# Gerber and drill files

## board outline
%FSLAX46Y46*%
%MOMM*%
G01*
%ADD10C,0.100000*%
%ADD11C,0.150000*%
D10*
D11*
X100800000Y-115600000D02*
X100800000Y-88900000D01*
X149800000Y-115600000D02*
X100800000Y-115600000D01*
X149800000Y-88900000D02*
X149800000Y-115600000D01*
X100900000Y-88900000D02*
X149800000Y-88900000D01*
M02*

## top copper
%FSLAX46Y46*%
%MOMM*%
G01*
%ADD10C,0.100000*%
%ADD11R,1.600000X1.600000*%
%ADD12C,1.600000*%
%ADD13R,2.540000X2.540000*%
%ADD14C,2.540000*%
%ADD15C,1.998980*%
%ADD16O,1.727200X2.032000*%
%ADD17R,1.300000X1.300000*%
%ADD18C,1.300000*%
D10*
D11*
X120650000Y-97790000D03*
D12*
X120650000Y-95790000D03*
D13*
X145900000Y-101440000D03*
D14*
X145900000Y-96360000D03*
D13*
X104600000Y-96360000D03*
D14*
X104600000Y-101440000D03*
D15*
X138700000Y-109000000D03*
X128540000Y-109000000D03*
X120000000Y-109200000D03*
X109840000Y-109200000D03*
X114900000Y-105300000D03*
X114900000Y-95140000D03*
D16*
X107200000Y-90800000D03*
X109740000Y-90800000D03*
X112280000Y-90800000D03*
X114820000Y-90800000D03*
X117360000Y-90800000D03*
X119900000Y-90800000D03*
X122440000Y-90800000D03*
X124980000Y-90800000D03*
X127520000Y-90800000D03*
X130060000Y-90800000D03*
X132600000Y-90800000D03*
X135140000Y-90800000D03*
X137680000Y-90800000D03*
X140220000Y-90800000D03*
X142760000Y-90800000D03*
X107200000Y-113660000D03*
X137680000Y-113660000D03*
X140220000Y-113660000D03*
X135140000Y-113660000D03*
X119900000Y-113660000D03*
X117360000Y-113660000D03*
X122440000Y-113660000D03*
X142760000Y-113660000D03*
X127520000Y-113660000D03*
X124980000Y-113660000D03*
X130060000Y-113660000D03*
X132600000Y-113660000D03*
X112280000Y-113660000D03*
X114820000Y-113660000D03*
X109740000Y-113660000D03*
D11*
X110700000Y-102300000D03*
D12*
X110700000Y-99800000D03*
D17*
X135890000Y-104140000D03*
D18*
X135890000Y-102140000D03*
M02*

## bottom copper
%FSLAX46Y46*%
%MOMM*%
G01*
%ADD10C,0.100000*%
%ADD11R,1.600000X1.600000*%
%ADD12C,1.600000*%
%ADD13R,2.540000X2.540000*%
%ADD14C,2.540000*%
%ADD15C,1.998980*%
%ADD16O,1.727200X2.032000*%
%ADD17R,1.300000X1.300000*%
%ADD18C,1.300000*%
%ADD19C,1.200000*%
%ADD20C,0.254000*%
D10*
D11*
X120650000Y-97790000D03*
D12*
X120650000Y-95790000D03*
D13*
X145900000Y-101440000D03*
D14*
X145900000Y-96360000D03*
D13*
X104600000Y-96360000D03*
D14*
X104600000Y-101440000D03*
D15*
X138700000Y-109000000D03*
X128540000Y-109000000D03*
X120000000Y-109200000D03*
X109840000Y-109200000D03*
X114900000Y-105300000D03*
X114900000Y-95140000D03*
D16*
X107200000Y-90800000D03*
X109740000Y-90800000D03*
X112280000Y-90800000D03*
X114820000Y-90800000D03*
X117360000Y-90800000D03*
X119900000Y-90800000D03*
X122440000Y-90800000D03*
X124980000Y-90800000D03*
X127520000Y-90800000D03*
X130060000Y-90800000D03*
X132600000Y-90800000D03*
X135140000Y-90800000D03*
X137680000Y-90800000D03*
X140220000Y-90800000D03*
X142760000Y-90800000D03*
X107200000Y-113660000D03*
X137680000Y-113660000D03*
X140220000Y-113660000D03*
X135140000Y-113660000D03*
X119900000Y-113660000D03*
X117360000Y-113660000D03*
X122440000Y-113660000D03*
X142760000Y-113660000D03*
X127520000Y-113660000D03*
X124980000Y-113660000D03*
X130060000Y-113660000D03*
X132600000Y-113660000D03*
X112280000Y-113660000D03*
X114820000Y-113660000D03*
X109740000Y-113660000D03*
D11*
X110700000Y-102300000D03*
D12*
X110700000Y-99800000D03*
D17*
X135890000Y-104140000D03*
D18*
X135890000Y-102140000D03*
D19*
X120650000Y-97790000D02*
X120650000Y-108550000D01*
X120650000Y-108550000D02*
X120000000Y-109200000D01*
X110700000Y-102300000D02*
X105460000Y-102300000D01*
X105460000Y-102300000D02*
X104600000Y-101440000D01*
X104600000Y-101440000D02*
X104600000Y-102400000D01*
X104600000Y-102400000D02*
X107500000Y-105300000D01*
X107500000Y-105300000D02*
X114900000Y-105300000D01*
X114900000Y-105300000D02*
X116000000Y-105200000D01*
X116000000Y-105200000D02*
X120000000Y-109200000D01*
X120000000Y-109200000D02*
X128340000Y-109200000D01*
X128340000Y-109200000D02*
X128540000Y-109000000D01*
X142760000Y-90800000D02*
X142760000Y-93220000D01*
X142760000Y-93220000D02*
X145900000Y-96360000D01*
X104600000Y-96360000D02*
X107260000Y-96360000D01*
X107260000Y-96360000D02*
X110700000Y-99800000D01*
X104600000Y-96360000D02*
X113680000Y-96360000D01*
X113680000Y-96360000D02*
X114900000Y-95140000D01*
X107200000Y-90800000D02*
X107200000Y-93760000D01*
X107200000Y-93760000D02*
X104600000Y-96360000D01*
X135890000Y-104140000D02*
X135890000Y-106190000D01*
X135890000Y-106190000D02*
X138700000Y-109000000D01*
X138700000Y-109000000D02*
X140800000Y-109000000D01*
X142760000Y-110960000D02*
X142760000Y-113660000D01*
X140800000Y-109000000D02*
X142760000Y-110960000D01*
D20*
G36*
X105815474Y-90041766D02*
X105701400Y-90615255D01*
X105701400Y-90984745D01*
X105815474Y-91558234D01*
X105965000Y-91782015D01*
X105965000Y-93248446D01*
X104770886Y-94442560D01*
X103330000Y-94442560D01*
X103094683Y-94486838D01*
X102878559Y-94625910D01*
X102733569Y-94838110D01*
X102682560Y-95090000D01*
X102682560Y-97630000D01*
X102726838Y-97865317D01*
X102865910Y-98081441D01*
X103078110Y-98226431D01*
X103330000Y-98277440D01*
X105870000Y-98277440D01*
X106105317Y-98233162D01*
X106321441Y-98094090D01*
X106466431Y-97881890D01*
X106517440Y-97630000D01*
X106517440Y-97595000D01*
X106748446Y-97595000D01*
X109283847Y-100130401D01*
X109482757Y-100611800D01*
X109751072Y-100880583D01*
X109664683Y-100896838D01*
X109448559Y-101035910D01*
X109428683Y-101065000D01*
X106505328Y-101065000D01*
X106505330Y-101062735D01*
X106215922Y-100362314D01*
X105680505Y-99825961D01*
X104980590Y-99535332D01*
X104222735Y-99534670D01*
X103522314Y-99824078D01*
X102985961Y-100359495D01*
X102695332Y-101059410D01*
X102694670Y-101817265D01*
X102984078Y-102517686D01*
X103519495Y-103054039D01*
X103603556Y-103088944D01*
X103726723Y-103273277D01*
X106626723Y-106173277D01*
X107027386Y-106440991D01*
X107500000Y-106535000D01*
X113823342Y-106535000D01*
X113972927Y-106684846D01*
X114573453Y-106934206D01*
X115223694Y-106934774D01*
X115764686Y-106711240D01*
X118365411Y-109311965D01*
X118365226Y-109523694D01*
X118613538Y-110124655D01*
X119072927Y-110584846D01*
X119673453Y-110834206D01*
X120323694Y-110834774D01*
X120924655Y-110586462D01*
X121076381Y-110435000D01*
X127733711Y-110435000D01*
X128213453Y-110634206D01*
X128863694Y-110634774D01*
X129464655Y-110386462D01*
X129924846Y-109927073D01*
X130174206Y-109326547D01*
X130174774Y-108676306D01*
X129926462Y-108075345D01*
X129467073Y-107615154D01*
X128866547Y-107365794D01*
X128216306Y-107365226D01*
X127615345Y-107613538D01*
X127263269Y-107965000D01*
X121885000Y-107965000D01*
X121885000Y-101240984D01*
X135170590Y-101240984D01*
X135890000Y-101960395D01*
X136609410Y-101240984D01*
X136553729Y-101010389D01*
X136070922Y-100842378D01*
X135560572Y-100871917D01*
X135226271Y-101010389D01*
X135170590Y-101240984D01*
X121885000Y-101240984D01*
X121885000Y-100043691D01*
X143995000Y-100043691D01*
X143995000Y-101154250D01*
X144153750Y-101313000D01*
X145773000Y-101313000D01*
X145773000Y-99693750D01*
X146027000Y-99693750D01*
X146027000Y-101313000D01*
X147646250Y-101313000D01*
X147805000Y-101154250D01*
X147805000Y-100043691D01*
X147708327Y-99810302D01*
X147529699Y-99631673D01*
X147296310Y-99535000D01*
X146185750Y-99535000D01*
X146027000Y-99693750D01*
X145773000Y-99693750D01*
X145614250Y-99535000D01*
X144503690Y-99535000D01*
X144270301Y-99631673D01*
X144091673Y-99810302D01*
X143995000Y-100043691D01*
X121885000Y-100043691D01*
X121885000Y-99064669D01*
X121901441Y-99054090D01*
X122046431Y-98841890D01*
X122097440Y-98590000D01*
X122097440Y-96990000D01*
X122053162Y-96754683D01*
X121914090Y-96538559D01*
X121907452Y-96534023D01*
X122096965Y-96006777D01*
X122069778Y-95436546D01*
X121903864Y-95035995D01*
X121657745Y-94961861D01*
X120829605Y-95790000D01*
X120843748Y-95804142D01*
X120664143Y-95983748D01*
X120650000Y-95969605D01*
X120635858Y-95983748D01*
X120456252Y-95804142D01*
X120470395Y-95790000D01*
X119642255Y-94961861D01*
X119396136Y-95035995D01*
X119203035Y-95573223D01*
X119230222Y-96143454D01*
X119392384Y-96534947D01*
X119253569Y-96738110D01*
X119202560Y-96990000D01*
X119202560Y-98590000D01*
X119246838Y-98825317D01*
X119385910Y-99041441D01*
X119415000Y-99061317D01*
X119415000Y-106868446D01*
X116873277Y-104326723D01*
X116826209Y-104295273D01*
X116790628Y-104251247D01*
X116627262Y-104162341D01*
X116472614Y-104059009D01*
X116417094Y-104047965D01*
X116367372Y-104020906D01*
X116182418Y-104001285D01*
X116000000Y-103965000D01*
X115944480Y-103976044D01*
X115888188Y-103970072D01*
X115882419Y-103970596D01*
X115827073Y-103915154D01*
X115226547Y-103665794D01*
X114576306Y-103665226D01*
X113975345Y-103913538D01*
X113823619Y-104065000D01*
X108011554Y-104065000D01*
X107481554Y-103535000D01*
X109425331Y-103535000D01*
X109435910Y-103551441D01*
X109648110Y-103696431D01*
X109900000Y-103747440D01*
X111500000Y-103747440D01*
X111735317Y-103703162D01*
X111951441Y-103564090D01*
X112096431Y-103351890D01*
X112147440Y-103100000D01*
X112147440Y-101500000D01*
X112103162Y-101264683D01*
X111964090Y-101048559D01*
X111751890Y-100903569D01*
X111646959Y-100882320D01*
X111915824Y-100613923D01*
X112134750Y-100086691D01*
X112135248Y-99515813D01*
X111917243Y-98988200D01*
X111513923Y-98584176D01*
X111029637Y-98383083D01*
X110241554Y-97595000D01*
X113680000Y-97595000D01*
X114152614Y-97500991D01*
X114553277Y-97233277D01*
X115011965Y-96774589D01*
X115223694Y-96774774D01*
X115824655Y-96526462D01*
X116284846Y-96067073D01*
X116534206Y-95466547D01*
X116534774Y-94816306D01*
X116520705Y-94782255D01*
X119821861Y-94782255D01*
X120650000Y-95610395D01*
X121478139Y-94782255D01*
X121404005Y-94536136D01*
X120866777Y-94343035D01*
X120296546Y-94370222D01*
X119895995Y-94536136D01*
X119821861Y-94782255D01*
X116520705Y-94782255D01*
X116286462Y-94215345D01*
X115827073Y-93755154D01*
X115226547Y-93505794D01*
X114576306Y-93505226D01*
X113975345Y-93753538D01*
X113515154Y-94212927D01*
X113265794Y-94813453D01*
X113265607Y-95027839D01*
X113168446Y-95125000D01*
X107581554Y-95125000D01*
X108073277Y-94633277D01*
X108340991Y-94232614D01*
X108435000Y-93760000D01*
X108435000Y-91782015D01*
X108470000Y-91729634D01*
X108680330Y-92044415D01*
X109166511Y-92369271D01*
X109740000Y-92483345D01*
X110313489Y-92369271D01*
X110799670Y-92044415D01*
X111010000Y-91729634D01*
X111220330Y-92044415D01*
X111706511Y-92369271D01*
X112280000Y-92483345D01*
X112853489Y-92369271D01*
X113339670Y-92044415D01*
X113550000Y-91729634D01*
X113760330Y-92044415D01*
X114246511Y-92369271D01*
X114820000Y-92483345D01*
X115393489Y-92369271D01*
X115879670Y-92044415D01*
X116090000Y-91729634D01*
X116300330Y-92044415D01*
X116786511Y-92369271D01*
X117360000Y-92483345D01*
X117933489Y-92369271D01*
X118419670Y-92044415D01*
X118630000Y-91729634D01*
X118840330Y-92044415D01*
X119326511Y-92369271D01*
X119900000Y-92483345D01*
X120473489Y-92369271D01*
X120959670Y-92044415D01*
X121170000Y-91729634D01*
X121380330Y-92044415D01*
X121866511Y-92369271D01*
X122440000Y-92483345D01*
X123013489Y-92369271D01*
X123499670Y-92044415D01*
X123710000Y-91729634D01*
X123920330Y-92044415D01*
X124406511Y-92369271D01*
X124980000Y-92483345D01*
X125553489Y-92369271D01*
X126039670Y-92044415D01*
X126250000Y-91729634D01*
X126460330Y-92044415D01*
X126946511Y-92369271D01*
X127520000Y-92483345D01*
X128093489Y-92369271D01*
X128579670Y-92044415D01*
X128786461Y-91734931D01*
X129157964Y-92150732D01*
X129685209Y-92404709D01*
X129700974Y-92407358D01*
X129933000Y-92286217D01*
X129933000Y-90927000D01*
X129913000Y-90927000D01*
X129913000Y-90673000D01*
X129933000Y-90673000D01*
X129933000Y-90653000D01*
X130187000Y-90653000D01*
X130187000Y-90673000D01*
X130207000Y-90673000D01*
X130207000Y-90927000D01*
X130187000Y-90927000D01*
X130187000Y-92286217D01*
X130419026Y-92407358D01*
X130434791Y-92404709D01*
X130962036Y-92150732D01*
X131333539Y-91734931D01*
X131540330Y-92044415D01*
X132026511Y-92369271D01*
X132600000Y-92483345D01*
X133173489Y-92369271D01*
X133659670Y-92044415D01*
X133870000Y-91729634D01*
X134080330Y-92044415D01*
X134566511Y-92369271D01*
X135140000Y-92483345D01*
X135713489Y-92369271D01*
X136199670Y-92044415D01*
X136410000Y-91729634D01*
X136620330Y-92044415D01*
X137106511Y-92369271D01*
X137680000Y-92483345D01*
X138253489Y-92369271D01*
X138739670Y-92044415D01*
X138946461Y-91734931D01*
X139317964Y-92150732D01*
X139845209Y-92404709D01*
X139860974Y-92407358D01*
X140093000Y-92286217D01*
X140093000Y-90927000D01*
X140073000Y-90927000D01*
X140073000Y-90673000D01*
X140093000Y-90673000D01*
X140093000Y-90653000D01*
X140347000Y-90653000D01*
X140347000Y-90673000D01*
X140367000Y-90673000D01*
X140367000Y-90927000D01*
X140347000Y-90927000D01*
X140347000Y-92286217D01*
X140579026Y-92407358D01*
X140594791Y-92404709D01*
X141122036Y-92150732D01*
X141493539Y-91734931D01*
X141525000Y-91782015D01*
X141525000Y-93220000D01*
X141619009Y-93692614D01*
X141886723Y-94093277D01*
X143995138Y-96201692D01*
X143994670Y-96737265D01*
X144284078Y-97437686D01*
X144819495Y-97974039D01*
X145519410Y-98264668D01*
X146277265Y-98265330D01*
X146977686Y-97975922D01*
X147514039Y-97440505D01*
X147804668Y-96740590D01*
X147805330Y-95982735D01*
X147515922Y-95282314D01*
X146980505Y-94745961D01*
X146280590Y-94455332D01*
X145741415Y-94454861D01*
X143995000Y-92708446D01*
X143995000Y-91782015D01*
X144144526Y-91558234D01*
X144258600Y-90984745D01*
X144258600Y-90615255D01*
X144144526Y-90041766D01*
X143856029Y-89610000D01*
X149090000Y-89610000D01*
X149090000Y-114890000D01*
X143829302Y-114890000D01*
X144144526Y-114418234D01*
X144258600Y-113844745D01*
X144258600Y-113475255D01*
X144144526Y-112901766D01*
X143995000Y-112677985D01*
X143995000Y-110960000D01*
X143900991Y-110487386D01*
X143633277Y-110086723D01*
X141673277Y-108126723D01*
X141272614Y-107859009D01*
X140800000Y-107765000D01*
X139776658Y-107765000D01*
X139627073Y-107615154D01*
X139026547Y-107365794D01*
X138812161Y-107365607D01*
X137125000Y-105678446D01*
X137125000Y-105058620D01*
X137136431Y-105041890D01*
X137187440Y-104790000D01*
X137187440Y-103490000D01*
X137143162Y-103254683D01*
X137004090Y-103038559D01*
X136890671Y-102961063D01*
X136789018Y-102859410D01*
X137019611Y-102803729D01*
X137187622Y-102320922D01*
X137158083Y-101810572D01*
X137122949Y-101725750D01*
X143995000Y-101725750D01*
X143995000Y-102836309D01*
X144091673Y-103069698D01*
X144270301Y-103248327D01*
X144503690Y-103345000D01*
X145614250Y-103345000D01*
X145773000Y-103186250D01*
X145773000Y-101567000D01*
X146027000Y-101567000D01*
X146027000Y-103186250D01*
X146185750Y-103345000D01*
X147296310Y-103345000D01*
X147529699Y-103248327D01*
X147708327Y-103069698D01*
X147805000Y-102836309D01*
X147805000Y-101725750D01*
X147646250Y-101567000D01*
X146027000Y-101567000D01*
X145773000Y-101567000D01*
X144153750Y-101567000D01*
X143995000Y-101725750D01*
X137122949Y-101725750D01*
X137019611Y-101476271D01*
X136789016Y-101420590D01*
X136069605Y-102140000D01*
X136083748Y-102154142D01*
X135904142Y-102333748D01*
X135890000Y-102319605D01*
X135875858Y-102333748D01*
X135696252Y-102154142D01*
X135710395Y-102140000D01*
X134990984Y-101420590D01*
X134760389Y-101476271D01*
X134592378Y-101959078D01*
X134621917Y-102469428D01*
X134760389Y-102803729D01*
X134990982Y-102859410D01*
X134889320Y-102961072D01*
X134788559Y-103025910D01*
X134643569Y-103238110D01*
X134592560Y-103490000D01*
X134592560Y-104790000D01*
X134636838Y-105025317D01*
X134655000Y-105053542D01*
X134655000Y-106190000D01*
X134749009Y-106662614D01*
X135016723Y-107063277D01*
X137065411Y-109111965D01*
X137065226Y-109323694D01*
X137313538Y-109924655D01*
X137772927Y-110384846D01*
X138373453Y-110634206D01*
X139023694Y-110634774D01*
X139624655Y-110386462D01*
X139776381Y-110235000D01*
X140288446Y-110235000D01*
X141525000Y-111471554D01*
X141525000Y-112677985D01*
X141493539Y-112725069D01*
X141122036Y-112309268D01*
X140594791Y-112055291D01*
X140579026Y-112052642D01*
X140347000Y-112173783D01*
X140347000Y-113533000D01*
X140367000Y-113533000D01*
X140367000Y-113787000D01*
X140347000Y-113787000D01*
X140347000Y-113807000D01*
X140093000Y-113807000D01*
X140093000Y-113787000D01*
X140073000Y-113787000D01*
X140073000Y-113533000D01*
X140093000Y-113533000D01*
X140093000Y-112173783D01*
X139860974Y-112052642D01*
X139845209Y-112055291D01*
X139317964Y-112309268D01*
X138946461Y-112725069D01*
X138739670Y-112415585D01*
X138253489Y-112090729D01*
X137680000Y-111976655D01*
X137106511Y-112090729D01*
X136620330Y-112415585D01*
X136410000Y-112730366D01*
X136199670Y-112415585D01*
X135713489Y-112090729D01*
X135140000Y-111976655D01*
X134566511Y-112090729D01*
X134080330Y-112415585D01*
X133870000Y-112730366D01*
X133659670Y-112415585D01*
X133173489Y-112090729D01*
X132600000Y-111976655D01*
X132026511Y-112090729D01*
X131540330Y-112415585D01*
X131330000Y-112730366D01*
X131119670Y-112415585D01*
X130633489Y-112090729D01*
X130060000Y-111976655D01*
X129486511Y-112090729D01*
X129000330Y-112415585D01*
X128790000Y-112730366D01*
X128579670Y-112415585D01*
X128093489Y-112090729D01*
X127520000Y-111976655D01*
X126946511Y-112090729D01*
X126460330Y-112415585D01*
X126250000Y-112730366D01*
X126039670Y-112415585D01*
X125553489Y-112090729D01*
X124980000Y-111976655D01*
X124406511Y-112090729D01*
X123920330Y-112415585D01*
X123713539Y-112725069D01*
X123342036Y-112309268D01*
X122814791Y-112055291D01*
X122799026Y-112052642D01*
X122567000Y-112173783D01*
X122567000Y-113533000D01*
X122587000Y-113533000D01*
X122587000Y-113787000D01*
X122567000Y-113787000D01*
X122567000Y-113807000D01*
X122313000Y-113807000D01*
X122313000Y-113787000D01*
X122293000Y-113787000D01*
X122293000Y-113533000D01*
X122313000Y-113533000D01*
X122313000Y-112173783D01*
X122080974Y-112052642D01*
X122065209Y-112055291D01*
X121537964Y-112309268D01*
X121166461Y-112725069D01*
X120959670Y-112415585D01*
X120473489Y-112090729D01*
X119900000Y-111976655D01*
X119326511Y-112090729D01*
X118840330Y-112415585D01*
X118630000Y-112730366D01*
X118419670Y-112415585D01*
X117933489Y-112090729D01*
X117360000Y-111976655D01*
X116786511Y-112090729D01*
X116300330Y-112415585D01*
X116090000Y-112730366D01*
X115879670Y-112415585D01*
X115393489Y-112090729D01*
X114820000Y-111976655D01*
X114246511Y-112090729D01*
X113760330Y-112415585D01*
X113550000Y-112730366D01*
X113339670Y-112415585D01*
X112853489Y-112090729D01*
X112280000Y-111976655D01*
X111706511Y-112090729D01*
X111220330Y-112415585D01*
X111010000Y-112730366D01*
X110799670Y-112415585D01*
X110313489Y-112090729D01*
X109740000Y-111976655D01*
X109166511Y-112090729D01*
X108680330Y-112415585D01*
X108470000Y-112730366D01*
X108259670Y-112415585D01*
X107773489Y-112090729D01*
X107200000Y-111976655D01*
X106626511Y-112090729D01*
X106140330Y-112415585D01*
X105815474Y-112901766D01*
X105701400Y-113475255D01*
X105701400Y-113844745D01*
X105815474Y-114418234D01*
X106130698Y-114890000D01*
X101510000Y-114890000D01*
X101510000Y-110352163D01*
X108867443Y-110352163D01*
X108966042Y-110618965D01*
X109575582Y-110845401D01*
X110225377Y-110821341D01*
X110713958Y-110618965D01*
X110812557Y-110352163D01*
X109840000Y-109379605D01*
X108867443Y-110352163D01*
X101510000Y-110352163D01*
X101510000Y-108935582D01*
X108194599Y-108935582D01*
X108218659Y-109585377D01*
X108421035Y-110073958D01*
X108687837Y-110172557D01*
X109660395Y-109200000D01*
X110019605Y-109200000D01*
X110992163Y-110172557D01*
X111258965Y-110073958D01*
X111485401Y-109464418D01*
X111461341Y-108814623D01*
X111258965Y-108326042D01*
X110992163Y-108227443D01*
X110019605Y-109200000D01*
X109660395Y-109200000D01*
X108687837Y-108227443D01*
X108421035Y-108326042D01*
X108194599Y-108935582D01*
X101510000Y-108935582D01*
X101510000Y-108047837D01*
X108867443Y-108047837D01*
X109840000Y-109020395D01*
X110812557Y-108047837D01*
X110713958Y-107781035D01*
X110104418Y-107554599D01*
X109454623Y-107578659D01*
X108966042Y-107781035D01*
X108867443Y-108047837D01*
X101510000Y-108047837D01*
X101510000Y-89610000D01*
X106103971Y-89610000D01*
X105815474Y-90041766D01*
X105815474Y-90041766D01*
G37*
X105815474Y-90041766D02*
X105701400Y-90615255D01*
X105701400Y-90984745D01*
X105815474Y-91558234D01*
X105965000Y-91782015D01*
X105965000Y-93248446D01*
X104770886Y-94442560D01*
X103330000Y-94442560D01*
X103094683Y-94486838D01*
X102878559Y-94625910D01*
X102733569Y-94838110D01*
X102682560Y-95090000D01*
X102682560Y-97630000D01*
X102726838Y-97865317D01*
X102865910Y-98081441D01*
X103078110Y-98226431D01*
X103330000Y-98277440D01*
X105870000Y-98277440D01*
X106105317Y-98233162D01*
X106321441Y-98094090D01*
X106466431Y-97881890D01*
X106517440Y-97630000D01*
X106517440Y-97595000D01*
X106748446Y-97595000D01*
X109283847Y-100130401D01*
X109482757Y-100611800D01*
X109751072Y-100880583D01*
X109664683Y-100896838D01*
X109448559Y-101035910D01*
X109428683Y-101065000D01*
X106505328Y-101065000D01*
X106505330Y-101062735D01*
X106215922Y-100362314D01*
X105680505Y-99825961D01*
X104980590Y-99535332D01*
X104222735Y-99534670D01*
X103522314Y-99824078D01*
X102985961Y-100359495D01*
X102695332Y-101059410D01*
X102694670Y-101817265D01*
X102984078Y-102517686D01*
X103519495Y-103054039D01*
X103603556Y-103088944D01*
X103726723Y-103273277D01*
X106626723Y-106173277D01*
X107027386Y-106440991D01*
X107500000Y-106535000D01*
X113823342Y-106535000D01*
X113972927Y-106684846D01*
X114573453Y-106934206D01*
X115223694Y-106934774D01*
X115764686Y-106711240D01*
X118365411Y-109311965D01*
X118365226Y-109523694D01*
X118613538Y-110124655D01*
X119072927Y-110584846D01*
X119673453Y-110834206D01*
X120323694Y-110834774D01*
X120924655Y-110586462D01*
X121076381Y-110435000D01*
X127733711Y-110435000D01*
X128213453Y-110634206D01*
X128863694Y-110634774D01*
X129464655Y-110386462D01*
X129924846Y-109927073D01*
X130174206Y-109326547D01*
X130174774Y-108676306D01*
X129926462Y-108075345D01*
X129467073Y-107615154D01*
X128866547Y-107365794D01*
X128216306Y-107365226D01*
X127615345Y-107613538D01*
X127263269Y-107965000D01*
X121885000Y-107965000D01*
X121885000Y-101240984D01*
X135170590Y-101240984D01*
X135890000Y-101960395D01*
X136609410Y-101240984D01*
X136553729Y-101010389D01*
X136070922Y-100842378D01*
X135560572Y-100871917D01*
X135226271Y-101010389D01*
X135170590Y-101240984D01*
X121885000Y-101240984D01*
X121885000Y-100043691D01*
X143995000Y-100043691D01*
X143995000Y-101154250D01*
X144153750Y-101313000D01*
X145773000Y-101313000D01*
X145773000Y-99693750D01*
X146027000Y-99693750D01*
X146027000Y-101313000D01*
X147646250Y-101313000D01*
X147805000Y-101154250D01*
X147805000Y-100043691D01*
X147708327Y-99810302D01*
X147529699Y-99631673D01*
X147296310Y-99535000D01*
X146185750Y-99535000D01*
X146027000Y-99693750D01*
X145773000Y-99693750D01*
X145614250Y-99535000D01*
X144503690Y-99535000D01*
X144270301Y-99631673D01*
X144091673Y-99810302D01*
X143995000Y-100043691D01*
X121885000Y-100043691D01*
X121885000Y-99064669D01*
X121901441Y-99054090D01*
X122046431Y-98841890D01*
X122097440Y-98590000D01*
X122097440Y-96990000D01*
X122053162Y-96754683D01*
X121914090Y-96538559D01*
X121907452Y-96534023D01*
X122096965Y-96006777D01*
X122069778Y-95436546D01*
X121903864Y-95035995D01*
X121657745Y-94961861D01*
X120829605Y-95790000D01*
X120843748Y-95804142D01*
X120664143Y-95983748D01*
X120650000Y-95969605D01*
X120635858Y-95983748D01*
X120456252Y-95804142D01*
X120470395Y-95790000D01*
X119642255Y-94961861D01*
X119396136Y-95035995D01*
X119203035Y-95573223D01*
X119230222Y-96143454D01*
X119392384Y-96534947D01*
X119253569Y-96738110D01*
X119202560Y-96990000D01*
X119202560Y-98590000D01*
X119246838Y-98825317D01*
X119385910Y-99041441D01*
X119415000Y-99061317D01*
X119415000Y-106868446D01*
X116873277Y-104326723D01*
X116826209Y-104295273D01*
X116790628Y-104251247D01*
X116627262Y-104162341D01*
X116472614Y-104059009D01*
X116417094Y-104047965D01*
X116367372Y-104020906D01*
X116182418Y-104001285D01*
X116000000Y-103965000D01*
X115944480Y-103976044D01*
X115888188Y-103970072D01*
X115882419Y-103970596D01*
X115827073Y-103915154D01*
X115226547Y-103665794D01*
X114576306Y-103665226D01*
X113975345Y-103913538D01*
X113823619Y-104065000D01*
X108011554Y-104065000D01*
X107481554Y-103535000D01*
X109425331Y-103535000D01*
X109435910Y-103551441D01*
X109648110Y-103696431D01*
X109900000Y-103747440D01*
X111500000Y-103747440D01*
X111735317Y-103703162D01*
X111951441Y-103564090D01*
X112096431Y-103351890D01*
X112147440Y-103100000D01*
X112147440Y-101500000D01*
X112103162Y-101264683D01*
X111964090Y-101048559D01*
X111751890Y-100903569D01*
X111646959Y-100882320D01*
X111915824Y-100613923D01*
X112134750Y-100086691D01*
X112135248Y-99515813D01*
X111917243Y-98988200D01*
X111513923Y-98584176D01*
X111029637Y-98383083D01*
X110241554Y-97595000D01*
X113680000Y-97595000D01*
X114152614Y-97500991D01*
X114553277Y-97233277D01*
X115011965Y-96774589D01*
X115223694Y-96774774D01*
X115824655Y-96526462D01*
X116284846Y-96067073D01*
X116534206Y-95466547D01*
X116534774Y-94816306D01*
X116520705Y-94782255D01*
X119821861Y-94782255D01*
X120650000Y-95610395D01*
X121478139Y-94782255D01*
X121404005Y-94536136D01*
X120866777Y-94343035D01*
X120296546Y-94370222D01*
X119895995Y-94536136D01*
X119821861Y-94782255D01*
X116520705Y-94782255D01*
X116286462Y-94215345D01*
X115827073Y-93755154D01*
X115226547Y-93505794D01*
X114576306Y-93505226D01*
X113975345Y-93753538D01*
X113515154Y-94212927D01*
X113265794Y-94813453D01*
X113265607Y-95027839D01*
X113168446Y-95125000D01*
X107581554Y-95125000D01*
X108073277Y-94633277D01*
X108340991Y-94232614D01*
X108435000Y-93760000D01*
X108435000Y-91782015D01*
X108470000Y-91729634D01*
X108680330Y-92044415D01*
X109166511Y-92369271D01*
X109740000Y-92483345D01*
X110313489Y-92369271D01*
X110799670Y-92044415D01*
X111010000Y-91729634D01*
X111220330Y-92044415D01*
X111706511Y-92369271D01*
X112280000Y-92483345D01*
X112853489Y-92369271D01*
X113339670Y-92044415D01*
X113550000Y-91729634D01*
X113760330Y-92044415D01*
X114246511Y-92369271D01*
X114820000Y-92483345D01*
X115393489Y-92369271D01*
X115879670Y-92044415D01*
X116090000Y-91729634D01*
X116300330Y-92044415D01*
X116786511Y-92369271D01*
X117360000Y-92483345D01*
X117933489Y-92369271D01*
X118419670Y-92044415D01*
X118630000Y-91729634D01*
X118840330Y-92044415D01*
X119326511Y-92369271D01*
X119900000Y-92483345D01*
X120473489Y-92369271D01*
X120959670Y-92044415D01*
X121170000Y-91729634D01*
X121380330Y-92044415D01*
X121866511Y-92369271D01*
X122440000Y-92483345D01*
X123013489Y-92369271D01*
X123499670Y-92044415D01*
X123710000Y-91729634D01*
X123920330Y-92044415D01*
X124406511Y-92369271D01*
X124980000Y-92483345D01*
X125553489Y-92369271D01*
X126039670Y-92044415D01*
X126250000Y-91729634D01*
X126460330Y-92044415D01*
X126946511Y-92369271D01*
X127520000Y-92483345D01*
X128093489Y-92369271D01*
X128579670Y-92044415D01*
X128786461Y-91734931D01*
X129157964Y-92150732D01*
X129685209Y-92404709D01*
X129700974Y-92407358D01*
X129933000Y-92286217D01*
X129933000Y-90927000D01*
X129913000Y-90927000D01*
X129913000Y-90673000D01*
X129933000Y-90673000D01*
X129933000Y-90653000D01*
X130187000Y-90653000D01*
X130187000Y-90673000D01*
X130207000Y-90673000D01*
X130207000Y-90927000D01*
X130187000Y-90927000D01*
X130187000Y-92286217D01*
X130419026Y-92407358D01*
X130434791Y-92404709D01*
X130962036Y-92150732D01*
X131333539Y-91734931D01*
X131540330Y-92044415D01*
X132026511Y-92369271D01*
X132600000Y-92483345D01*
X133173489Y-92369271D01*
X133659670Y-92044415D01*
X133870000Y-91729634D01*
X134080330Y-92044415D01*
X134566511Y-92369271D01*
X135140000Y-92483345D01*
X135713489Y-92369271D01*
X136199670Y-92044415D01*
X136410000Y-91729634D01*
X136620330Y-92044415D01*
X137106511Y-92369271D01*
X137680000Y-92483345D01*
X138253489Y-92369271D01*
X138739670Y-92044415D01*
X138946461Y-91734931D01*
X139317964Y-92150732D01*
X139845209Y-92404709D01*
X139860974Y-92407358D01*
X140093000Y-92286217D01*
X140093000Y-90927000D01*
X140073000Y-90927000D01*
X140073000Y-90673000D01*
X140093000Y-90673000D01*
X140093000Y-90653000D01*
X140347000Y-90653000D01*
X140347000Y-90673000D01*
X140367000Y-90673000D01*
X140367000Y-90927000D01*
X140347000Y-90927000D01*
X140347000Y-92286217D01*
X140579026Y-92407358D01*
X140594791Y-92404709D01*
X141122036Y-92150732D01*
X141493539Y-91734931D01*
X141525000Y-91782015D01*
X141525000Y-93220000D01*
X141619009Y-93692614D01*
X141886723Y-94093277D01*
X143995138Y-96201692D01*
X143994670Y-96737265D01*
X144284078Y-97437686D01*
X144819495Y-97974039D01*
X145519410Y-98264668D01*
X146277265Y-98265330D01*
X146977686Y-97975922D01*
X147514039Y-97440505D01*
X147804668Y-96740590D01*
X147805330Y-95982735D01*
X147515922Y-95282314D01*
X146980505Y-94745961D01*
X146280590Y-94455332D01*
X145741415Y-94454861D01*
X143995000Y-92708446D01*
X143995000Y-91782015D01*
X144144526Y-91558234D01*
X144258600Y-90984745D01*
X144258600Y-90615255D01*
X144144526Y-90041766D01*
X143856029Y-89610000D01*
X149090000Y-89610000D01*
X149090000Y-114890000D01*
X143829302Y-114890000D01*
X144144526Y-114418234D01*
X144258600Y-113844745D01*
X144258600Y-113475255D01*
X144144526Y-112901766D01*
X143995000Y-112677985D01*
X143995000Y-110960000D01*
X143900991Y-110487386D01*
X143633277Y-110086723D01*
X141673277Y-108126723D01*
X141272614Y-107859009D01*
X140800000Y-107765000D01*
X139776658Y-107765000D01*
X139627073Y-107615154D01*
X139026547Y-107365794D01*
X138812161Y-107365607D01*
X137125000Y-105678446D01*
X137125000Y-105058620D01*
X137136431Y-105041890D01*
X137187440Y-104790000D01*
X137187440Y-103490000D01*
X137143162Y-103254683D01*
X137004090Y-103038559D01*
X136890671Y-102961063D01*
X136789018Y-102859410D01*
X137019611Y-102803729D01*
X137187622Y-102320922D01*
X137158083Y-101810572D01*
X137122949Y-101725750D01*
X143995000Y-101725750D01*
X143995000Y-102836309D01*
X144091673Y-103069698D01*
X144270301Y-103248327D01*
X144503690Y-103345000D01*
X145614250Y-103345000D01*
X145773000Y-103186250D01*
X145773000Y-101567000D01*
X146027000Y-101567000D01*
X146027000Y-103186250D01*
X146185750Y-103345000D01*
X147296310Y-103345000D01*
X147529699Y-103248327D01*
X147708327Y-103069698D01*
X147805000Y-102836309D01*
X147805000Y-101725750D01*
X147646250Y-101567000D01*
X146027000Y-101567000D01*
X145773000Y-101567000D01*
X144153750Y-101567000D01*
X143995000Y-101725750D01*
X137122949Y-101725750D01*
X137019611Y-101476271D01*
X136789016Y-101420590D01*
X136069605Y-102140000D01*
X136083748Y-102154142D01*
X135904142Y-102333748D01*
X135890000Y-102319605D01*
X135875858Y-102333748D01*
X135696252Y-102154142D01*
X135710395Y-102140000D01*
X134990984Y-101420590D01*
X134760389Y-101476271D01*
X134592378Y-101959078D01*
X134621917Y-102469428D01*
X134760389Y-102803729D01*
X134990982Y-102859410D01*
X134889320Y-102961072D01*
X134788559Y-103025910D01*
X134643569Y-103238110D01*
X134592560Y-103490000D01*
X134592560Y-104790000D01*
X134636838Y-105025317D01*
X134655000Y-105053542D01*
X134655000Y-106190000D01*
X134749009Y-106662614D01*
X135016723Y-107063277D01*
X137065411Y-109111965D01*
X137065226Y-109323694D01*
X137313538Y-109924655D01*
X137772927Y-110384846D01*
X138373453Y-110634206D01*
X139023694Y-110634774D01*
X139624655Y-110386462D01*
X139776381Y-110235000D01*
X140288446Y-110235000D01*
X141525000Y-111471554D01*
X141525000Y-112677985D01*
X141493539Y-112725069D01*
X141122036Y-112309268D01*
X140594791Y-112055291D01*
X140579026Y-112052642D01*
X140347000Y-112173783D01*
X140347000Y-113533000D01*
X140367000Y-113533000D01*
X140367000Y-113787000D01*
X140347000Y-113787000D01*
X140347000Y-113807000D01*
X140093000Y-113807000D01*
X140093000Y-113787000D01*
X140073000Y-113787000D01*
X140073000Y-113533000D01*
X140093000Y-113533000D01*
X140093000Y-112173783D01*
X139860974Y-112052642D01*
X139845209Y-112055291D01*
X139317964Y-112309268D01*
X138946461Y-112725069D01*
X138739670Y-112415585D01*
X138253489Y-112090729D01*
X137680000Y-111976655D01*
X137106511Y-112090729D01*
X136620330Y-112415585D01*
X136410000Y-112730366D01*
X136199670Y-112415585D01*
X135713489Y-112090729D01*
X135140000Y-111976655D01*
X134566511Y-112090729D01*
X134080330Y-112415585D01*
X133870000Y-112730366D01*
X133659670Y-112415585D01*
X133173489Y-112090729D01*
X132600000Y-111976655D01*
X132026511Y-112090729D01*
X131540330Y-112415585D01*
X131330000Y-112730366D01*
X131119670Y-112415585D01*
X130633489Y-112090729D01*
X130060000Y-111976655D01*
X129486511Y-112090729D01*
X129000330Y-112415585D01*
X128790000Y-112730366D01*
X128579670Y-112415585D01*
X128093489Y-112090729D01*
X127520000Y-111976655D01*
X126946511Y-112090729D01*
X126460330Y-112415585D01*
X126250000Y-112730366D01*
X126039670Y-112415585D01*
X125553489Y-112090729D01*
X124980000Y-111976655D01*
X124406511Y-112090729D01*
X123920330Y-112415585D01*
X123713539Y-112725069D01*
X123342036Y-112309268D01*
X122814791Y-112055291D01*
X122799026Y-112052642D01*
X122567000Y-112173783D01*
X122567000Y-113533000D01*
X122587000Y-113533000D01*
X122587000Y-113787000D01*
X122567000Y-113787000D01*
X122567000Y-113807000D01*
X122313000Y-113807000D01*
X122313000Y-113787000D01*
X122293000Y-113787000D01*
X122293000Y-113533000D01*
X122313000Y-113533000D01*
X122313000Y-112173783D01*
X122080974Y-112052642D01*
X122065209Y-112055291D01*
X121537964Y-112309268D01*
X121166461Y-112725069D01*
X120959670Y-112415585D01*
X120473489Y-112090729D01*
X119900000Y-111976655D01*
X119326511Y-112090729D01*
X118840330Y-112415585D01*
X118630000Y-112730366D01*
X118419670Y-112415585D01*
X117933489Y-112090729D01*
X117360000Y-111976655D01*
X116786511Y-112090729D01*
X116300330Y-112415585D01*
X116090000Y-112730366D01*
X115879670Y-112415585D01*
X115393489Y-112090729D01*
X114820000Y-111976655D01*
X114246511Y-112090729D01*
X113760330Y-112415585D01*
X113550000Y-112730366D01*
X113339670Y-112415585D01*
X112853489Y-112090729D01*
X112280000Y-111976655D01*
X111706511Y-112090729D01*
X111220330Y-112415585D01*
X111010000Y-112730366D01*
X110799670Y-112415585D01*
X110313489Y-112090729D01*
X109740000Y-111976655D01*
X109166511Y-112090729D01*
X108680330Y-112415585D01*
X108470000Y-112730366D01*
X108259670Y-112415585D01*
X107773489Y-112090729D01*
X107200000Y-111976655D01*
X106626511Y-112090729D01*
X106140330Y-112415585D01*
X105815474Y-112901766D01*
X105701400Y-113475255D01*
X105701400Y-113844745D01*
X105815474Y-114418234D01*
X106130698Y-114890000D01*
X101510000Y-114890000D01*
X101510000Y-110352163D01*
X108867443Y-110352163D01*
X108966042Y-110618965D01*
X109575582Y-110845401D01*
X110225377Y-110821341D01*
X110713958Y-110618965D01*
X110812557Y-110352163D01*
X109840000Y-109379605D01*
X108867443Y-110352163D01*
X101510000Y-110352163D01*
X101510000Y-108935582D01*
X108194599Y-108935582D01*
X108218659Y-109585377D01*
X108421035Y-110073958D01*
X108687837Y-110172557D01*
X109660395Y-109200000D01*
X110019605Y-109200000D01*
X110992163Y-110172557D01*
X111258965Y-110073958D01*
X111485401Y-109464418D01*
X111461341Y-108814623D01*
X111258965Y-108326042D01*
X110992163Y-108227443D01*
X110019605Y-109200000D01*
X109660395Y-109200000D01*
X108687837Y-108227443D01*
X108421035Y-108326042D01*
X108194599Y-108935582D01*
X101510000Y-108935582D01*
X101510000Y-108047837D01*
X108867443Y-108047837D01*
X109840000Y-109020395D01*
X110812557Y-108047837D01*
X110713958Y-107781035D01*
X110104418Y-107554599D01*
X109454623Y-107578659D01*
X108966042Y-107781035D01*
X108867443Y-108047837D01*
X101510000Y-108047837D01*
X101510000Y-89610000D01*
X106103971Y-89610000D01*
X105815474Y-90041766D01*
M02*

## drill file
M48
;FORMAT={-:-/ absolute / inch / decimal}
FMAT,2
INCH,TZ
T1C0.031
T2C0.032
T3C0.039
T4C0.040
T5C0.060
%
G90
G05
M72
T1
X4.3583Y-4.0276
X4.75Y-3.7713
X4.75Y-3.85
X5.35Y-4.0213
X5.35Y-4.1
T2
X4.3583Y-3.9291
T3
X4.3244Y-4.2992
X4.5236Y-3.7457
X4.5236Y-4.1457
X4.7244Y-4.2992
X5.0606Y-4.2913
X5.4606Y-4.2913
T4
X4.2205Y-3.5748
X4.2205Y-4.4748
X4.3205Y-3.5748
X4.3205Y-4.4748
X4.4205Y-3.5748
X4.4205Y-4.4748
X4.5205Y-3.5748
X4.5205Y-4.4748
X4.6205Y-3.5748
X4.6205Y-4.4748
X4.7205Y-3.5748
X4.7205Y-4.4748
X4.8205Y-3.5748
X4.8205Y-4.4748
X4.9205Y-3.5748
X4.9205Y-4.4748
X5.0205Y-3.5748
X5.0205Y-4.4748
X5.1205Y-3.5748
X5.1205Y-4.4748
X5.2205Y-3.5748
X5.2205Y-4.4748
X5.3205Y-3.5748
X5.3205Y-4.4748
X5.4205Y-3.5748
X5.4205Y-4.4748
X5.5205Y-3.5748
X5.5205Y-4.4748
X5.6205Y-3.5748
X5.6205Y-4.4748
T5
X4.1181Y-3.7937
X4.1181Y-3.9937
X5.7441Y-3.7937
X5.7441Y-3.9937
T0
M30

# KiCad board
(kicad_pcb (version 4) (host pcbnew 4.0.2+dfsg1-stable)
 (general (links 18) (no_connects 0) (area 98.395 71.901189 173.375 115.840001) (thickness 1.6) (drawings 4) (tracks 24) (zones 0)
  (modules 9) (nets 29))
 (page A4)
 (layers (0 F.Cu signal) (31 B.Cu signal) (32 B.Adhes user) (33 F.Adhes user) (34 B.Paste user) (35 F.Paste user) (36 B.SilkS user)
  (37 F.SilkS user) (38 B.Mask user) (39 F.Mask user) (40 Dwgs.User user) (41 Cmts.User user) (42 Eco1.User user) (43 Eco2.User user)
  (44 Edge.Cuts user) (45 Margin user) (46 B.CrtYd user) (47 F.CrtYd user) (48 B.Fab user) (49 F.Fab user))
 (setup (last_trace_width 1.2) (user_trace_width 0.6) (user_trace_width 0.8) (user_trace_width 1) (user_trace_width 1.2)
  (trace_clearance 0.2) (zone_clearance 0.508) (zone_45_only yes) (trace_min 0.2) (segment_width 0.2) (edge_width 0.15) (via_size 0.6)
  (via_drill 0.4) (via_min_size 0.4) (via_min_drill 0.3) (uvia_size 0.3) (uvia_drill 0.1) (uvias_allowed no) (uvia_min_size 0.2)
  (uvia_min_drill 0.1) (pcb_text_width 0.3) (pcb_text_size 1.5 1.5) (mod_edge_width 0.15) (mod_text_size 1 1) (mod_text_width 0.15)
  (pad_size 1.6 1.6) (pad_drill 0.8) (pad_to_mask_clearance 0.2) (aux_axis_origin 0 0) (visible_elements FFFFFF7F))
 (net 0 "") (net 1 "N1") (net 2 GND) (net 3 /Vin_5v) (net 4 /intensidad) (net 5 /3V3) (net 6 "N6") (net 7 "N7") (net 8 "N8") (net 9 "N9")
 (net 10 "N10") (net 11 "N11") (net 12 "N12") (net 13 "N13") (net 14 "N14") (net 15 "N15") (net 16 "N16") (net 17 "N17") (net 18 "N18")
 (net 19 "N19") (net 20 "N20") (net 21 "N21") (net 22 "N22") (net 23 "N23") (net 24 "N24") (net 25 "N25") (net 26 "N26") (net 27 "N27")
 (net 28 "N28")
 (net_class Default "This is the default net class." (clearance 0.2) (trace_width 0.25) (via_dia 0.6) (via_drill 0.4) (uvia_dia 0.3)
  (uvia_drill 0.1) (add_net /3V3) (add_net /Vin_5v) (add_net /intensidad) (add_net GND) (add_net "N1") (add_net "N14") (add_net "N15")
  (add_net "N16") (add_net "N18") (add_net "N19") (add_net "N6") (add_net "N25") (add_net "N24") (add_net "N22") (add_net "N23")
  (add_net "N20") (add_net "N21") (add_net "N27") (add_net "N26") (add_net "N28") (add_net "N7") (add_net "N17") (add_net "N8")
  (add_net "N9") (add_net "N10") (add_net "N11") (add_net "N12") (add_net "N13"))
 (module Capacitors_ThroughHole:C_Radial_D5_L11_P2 (layer F.Cu) (at 120.65 97.79 90)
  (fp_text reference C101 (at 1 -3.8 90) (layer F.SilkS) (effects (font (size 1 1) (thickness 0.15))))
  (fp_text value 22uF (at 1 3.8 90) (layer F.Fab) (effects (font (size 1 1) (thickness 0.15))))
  (pad 1 thru_hole rect (at 0 0 90) (size 1.6 1.6) (drill 0.8) (layers *.Cu *.Mask F.SilkS) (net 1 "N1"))
  (pad 2 thru_hole circle (at 2 0 90) (size 1.6 1.6) (drill 0.8) (layers *.Cu *.Mask F.SilkS) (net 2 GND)))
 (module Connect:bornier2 (layer F.Cu) (at 145.9 98.9 90)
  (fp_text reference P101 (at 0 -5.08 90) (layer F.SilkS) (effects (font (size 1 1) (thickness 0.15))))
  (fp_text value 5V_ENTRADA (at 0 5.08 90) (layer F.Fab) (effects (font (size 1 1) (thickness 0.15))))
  (pad 1 thru_hole rect (at -2.54 0 90) (size 2.54 2.54) (drill 1.524) (layers *.Cu *.Mask F.SilkS) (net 2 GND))
  (pad 2 thru_hole circle (at 2.54 0 90) (size 2.54 2.54) (drill 1.524) (layers *.Cu *.Mask F.SilkS) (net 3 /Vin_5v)))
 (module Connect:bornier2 (layer F.Cu) (at 104.6 98.9 270)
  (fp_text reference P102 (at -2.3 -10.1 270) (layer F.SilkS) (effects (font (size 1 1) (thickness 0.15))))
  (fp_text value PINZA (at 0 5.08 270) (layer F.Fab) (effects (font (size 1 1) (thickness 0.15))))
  (pad 1 thru_hole rect (at -2.54 0 270) (size 2.54 2.54) (drill 1.524) (layers *.Cu *.Mask F.SilkS) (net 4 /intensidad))
  (pad 2 thru_hole circle (at 2.54 0 270) (size 2.54 2.54) (drill 1.524) (layers *.Cu *.Mask F.SilkS) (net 1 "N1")))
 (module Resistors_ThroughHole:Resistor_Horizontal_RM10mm (layer F.Cu) (at 138.7 109 180)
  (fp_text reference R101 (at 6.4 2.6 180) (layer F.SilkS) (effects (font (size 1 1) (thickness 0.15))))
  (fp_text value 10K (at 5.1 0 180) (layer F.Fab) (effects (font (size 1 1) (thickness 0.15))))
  (pad 1 thru_hole circle (at 0 0 180) (size 1.99898 1.99898) (drill 1.00076) (layers *.Cu *.SilkS *.Mask) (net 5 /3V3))
  (pad 2 thru_hole circle (at 10.16 0 180) (size 1.99898 1.99898) (drill 1.00076) (layers *.Cu *.SilkS *.Mask) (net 1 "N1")))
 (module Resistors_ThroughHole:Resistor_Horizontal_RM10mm (layer F.Cu) (at 120 109.2 180)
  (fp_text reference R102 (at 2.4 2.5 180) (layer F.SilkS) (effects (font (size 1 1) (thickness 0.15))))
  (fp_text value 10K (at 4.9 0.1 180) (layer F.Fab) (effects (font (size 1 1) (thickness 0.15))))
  (pad 1 thru_hole circle (at 0 0 180) (size 1.99898 1.99898) (drill 1.00076) (layers *.Cu *.SilkS *.Mask) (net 1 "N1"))
  (pad 2 thru_hole circle (at 10.16 0 180) (size 1.99898 1.99898) (drill 1.00076) (layers *.Cu *.SilkS *.Mask) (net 2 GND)))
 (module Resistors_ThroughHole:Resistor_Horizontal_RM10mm (layer F.Cu) (at 114.9 105.3 90)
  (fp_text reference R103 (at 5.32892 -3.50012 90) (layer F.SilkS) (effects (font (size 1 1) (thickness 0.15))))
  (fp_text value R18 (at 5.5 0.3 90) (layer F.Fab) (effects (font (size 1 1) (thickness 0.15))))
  (pad 1 thru_hole circle (at 0 0 90) (size 1.99898 1.99898) (drill 1.00076) (layers *.Cu *.SilkS *.Mask) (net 1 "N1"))
  (pad 2 thru_hole circle (at 10.16 0 90) (size 1.99898 1.99898) (drill 1.00076) (layers *.Cu *.SilkS *.Mask) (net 4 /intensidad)))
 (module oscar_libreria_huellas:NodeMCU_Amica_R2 (layer B.Cu) (at 107.2 90.8 270)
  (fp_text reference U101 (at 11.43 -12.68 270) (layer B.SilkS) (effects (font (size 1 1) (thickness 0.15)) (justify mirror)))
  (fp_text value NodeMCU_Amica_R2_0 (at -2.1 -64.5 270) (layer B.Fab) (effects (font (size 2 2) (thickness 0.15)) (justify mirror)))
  (pad 1 thru_hole oval (at 0 0 270) (size 2.032 1.7272) (drill 1.016) (layers *.Cu *.Mask B.SilkS) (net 4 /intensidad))
  (pad 2 thru_hole oval (at 0 -2.54 270) (size 2.032 1.7272) (drill 1.016) (layers *.Cu *.Mask B.SilkS) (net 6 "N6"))
  (pad 3 thru_hole oval (at 0 -5.08 270) (size 2.032 1.7272) (drill 1.016) (layers *.Cu *.Mask B.SilkS) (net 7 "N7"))
  (pad 4 thru_hole oval (at 0 -7.62 270) (size 2.032 1.7272) (drill 1.016) (layers *.Cu *.Mask B.SilkS) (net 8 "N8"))
  (pad 5 thru_hole oval (at 0 -10.16 270) (size 2.032 1.7272) (drill 1.016) (layers *.Cu *.Mask B.SilkS) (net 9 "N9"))
  (pad 6 thru_hole oval (at 0 -12.7 270) (size 2.032 1.7272) (drill 1.016) (layers *.Cu *.Mask B.SilkS) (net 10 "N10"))
  (pad 7 thru_hole oval (at 0 -15.24 270) (size 2.032 1.7272) (drill 1.016) (layers *.Cu *.Mask B.SilkS) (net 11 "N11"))
  (pad 8 thru_hole oval (at 0 -17.78 270) (size 2.032 1.7272) (drill 1.016) (layers *.Cu *.Mask B.SilkS) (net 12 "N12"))
  (pad 9 thru_hole oval (at 0 -20.32 270) (size 2.032 1.7272) (drill 1.016) (layers *.Cu *.Mask B.SilkS) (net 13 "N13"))
  (pad 10 thru_hole oval (at 0 -22.86 270) (size 2.032 1.7272) (drill 1.016) (layers *.Cu *.Mask B.SilkS) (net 2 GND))
  (pad 11 thru_hole oval (at 0 -25.4 270) (size 2.032 1.7272) (drill 1.016) (layers *.Cu *.Mask B.SilkS) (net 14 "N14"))
  (pad 12 thru_hole oval (at 0 -27.94 270) (size 2.032 1.7272) (drill 1.016) (layers *.Cu *.Mask B.SilkS) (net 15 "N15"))
  (pad 13 thru_hole oval (at 0 -30.48 270) (size 2.032 1.7272) (drill 1.016) (layers *.Cu *.Mask B.SilkS) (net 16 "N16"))
  (pad 14 thru_hole oval (at 0 -33.02 270) (size 2.032 1.7272) (drill 1.016) (layers *.Cu *.Mask B.SilkS) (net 2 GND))
  (pad 15 thru_hole oval (at 0 -35.56 270) (size 2.032 1.7272) (drill 1.016) (layers *.Cu *.Mask B.SilkS) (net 3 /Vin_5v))
  (pad 30 thru_hole oval (at 22.86 0 270) (size 2.032 1.7272) (drill 1.016) (layers *.Cu *.Mask B.SilkS) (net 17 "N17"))
  (pad 18 thru_hole oval (at 22.86 -30.48 270) (size 2.032 1.7272) (drill 1.016) (layers *.Cu *.Mask B.SilkS) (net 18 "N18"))
  (pad 17 thru_hole oval (at 22.86 -33.02 270) (size 2.032 1.7272) (drill 1.016) (layers *.Cu *.Mask B.SilkS) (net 2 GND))
  (pad 19 thru_hole oval (at 22.86 -27.94 270) (size 2.032 1.7272) (drill 1.016) (layers *.Cu *.Mask B.SilkS) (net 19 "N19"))
  (pad 25 thru_hole oval (at 22.86 -12.7 270) (size 2.032 1.7272) (drill 1.016) (layers *.Cu *.Mask B.SilkS) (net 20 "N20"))
  (pad 26 thru_hole oval (at 22.86 -10.16 270) (size 2.032 1.7272) (drill 1.016) (layers *.Cu *.Mask B.SilkS) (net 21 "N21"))
  (pad 24 thru_hole oval (at 22.86 -15.24 270) (size 2.032 1.7272) (drill 1.016) (layers *.Cu *.Mask B.SilkS) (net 2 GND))
  (pad 16 thru_hole oval (at 22.86 -35.56 270) (size 2.032 1.7272) (drill 1.016) (layers *.Cu *.Mask B.SilkS) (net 5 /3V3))
  (pad 22 thru_hole oval (at 22.86 -20.32 270) (size 2.032 1.7272) (drill 1.016) (layers *.Cu *.Mask B.SilkS) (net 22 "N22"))
  (pad 23 thru_hole oval (at 22.86 -17.78 270) (size 2.032 1.7272) (drill 1.016) (layers *.Cu *.Mask B.SilkS) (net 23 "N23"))
  (pad 21 thru_hole oval (at 22.86 -22.86 270) (size 2.032 1.7272) (drill 1.016) (layers *.Cu *.Mask B.SilkS) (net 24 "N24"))
  (pad 20 thru_hole oval (at 22.86 -25.4 270) (size 2.032 1.7272) (drill 1.016) (layers *.Cu *.Mask B.SilkS) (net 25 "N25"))
  (pad 28 thru_hole oval (at 22.86 -5.08 270) (size 2.032 1.7272) (drill 1.016) (layers *.Cu *.Mask B.SilkS) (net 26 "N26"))
  (pad 27 thru_hole oval (at 22.86 -7.62 270) (size 2.032 1.7272) (drill 1.016) (layers *.Cu *.Mask B.SilkS) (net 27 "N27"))
  (pad 29 thru_hole oval (at 22.86 -2.54 270) (size 2.032 1.7272) (drill 1.016) (layers *.Cu *.Mask B.SilkS) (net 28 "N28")))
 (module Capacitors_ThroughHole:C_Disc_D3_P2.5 (layer F.Cu) (at 110.7 102.3 90)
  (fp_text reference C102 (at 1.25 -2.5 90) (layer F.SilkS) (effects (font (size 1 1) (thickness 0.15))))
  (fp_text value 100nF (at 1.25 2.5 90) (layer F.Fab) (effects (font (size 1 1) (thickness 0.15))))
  (pad 1 thru_hole rect (at 0 0 90) (size 1.6 1.6) (drill 0.8) (layers *.Cu *.Mask F.SilkS) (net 1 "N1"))
  (pad 2 thru_hole circle (at 2.5 0 90) (size 1.6 1.6) (drill 0.8001) (layers *.Cu *.Mask F.SilkS) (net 4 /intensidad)))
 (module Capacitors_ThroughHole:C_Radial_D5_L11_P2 (layer F.Cu) (at 135.89 104.14 90)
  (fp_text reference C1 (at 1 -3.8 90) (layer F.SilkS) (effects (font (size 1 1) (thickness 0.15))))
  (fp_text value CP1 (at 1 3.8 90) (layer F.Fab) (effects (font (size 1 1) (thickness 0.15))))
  (pad 1 thru_hole rect (at 0 0 90) (size 1.3 1.3) (drill 0.8) (layers *.Cu *.Mask F.SilkS) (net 5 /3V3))
  (pad 2 thru_hole circle (at 2 0 90) (size 1.3 1.3) (drill 0.8) (layers *.Cu *.Mask F.SilkS) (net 2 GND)))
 (gr_line (start 100.8 115.6) (end 100.8 88.9) (angle 90) (layer Edge.Cuts) (width 0.15))
 (gr_line (start 149.8 115.6) (end 100.8 115.6) (angle 90) (layer Edge.Cuts) (width 0.15))
 (gr_line (start 149.8 88.9) (end 149.8 115.6) (angle 90) (layer Edge.Cuts) (width 0.15))
 (gr_line (start 100.9 88.9) (end 149.8 88.9) (angle 90) (layer Edge.Cuts) (width 0.15))
 (segment (start 120.65 97.79) (end 120.65 108.55) (width 1.2) (layer B.Cu) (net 1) (status C00000))
 (segment (start 120.65 108.55) (end 120 109.2) (width 1.2) (layer B.Cu) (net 1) (status C00000))
 (segment (start 110.7 102.3) (end 105.46 102.3) (width 1.2) (layer B.Cu) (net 1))
 (segment (start 105.46 102.3) (end 104.6 101.44) (width 1.2) (layer B.Cu) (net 1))
 (segment (start 104.6 101.44) (end 104.6 102.4) (width 1.2) (layer B.Cu) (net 1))
 (segment (start 104.6 102.4) (end 107.5 105.3) (width 1.2) (layer B.Cu) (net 1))
 (segment (start 107.5 105.3) (end 114.9 105.3) (width 1.2) (layer B.Cu) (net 1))
 (segment (start 114.9 105.3) (end 116 105.2) (width 1.2) (layer B.Cu) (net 1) (status 10))
 (segment (start 116 105.2) (end 120 109.2) (width 1.2) (layer B.Cu) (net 1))
 (segment (start 120 109.2) (end 128.34 109.2) (width 1.2) (layer B.Cu) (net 1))
 (segment (start 128.34 109.2) (end 128.54 109) (width 1.2) (layer B.Cu) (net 1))
 (segment (start 142.76 90.8) (end 142.76 93.22) (width 1.2) (layer B.Cu) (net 3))
 (segment (start 142.76 93.22) (end 145.9 96.36) (width 1.2) (layer B.Cu) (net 3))
 (segment (start 104.6 96.36) (end 107.26 96.36) (width 1.2) (layer B.Cu) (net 4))
 (segment (start 107.26 96.36) (end 110.7 99.8) (width 1.2) (layer B.Cu) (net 4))
 (segment (start 104.6 96.36) (end 113.68 96.36) (width 1.2) (layer B.Cu) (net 4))
 (segment (start 113.68 96.36) (end 114.9 95.14) (width 1.2) (layer B.Cu) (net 4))
 (segment (start 107.2 90.8) (end 107.2 93.76) (width 1.2) (layer B.Cu) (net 4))
 (segment (start 107.2 93.76) (end 104.6 96.36) (width 1.2) (layer B.Cu) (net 4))
 (segment (start 135.89 104.14) (end 135.89 106.19) (width 1.2) (layer B.Cu) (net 5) (status 400000))
 (segment (start 135.89 106.19) (end 138.7 109) (width 1.2) (layer B.Cu) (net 5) (status 800000))
 (segment (start 138.7 109) (end 140.8 109) (width 1.2) (layer B.Cu) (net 5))
 (segment (start 142.76 110.96) (end 142.76 113.66) (width 1.2) (layer B.Cu) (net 5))
 (segment (start 140.8 109) (end 142.76 110.96) (width 1.2) (layer B.Cu) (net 5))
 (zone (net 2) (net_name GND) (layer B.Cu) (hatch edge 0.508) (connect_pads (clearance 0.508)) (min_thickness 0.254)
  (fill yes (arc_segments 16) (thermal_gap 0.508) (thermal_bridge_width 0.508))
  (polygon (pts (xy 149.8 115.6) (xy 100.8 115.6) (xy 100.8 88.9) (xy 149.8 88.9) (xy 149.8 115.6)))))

